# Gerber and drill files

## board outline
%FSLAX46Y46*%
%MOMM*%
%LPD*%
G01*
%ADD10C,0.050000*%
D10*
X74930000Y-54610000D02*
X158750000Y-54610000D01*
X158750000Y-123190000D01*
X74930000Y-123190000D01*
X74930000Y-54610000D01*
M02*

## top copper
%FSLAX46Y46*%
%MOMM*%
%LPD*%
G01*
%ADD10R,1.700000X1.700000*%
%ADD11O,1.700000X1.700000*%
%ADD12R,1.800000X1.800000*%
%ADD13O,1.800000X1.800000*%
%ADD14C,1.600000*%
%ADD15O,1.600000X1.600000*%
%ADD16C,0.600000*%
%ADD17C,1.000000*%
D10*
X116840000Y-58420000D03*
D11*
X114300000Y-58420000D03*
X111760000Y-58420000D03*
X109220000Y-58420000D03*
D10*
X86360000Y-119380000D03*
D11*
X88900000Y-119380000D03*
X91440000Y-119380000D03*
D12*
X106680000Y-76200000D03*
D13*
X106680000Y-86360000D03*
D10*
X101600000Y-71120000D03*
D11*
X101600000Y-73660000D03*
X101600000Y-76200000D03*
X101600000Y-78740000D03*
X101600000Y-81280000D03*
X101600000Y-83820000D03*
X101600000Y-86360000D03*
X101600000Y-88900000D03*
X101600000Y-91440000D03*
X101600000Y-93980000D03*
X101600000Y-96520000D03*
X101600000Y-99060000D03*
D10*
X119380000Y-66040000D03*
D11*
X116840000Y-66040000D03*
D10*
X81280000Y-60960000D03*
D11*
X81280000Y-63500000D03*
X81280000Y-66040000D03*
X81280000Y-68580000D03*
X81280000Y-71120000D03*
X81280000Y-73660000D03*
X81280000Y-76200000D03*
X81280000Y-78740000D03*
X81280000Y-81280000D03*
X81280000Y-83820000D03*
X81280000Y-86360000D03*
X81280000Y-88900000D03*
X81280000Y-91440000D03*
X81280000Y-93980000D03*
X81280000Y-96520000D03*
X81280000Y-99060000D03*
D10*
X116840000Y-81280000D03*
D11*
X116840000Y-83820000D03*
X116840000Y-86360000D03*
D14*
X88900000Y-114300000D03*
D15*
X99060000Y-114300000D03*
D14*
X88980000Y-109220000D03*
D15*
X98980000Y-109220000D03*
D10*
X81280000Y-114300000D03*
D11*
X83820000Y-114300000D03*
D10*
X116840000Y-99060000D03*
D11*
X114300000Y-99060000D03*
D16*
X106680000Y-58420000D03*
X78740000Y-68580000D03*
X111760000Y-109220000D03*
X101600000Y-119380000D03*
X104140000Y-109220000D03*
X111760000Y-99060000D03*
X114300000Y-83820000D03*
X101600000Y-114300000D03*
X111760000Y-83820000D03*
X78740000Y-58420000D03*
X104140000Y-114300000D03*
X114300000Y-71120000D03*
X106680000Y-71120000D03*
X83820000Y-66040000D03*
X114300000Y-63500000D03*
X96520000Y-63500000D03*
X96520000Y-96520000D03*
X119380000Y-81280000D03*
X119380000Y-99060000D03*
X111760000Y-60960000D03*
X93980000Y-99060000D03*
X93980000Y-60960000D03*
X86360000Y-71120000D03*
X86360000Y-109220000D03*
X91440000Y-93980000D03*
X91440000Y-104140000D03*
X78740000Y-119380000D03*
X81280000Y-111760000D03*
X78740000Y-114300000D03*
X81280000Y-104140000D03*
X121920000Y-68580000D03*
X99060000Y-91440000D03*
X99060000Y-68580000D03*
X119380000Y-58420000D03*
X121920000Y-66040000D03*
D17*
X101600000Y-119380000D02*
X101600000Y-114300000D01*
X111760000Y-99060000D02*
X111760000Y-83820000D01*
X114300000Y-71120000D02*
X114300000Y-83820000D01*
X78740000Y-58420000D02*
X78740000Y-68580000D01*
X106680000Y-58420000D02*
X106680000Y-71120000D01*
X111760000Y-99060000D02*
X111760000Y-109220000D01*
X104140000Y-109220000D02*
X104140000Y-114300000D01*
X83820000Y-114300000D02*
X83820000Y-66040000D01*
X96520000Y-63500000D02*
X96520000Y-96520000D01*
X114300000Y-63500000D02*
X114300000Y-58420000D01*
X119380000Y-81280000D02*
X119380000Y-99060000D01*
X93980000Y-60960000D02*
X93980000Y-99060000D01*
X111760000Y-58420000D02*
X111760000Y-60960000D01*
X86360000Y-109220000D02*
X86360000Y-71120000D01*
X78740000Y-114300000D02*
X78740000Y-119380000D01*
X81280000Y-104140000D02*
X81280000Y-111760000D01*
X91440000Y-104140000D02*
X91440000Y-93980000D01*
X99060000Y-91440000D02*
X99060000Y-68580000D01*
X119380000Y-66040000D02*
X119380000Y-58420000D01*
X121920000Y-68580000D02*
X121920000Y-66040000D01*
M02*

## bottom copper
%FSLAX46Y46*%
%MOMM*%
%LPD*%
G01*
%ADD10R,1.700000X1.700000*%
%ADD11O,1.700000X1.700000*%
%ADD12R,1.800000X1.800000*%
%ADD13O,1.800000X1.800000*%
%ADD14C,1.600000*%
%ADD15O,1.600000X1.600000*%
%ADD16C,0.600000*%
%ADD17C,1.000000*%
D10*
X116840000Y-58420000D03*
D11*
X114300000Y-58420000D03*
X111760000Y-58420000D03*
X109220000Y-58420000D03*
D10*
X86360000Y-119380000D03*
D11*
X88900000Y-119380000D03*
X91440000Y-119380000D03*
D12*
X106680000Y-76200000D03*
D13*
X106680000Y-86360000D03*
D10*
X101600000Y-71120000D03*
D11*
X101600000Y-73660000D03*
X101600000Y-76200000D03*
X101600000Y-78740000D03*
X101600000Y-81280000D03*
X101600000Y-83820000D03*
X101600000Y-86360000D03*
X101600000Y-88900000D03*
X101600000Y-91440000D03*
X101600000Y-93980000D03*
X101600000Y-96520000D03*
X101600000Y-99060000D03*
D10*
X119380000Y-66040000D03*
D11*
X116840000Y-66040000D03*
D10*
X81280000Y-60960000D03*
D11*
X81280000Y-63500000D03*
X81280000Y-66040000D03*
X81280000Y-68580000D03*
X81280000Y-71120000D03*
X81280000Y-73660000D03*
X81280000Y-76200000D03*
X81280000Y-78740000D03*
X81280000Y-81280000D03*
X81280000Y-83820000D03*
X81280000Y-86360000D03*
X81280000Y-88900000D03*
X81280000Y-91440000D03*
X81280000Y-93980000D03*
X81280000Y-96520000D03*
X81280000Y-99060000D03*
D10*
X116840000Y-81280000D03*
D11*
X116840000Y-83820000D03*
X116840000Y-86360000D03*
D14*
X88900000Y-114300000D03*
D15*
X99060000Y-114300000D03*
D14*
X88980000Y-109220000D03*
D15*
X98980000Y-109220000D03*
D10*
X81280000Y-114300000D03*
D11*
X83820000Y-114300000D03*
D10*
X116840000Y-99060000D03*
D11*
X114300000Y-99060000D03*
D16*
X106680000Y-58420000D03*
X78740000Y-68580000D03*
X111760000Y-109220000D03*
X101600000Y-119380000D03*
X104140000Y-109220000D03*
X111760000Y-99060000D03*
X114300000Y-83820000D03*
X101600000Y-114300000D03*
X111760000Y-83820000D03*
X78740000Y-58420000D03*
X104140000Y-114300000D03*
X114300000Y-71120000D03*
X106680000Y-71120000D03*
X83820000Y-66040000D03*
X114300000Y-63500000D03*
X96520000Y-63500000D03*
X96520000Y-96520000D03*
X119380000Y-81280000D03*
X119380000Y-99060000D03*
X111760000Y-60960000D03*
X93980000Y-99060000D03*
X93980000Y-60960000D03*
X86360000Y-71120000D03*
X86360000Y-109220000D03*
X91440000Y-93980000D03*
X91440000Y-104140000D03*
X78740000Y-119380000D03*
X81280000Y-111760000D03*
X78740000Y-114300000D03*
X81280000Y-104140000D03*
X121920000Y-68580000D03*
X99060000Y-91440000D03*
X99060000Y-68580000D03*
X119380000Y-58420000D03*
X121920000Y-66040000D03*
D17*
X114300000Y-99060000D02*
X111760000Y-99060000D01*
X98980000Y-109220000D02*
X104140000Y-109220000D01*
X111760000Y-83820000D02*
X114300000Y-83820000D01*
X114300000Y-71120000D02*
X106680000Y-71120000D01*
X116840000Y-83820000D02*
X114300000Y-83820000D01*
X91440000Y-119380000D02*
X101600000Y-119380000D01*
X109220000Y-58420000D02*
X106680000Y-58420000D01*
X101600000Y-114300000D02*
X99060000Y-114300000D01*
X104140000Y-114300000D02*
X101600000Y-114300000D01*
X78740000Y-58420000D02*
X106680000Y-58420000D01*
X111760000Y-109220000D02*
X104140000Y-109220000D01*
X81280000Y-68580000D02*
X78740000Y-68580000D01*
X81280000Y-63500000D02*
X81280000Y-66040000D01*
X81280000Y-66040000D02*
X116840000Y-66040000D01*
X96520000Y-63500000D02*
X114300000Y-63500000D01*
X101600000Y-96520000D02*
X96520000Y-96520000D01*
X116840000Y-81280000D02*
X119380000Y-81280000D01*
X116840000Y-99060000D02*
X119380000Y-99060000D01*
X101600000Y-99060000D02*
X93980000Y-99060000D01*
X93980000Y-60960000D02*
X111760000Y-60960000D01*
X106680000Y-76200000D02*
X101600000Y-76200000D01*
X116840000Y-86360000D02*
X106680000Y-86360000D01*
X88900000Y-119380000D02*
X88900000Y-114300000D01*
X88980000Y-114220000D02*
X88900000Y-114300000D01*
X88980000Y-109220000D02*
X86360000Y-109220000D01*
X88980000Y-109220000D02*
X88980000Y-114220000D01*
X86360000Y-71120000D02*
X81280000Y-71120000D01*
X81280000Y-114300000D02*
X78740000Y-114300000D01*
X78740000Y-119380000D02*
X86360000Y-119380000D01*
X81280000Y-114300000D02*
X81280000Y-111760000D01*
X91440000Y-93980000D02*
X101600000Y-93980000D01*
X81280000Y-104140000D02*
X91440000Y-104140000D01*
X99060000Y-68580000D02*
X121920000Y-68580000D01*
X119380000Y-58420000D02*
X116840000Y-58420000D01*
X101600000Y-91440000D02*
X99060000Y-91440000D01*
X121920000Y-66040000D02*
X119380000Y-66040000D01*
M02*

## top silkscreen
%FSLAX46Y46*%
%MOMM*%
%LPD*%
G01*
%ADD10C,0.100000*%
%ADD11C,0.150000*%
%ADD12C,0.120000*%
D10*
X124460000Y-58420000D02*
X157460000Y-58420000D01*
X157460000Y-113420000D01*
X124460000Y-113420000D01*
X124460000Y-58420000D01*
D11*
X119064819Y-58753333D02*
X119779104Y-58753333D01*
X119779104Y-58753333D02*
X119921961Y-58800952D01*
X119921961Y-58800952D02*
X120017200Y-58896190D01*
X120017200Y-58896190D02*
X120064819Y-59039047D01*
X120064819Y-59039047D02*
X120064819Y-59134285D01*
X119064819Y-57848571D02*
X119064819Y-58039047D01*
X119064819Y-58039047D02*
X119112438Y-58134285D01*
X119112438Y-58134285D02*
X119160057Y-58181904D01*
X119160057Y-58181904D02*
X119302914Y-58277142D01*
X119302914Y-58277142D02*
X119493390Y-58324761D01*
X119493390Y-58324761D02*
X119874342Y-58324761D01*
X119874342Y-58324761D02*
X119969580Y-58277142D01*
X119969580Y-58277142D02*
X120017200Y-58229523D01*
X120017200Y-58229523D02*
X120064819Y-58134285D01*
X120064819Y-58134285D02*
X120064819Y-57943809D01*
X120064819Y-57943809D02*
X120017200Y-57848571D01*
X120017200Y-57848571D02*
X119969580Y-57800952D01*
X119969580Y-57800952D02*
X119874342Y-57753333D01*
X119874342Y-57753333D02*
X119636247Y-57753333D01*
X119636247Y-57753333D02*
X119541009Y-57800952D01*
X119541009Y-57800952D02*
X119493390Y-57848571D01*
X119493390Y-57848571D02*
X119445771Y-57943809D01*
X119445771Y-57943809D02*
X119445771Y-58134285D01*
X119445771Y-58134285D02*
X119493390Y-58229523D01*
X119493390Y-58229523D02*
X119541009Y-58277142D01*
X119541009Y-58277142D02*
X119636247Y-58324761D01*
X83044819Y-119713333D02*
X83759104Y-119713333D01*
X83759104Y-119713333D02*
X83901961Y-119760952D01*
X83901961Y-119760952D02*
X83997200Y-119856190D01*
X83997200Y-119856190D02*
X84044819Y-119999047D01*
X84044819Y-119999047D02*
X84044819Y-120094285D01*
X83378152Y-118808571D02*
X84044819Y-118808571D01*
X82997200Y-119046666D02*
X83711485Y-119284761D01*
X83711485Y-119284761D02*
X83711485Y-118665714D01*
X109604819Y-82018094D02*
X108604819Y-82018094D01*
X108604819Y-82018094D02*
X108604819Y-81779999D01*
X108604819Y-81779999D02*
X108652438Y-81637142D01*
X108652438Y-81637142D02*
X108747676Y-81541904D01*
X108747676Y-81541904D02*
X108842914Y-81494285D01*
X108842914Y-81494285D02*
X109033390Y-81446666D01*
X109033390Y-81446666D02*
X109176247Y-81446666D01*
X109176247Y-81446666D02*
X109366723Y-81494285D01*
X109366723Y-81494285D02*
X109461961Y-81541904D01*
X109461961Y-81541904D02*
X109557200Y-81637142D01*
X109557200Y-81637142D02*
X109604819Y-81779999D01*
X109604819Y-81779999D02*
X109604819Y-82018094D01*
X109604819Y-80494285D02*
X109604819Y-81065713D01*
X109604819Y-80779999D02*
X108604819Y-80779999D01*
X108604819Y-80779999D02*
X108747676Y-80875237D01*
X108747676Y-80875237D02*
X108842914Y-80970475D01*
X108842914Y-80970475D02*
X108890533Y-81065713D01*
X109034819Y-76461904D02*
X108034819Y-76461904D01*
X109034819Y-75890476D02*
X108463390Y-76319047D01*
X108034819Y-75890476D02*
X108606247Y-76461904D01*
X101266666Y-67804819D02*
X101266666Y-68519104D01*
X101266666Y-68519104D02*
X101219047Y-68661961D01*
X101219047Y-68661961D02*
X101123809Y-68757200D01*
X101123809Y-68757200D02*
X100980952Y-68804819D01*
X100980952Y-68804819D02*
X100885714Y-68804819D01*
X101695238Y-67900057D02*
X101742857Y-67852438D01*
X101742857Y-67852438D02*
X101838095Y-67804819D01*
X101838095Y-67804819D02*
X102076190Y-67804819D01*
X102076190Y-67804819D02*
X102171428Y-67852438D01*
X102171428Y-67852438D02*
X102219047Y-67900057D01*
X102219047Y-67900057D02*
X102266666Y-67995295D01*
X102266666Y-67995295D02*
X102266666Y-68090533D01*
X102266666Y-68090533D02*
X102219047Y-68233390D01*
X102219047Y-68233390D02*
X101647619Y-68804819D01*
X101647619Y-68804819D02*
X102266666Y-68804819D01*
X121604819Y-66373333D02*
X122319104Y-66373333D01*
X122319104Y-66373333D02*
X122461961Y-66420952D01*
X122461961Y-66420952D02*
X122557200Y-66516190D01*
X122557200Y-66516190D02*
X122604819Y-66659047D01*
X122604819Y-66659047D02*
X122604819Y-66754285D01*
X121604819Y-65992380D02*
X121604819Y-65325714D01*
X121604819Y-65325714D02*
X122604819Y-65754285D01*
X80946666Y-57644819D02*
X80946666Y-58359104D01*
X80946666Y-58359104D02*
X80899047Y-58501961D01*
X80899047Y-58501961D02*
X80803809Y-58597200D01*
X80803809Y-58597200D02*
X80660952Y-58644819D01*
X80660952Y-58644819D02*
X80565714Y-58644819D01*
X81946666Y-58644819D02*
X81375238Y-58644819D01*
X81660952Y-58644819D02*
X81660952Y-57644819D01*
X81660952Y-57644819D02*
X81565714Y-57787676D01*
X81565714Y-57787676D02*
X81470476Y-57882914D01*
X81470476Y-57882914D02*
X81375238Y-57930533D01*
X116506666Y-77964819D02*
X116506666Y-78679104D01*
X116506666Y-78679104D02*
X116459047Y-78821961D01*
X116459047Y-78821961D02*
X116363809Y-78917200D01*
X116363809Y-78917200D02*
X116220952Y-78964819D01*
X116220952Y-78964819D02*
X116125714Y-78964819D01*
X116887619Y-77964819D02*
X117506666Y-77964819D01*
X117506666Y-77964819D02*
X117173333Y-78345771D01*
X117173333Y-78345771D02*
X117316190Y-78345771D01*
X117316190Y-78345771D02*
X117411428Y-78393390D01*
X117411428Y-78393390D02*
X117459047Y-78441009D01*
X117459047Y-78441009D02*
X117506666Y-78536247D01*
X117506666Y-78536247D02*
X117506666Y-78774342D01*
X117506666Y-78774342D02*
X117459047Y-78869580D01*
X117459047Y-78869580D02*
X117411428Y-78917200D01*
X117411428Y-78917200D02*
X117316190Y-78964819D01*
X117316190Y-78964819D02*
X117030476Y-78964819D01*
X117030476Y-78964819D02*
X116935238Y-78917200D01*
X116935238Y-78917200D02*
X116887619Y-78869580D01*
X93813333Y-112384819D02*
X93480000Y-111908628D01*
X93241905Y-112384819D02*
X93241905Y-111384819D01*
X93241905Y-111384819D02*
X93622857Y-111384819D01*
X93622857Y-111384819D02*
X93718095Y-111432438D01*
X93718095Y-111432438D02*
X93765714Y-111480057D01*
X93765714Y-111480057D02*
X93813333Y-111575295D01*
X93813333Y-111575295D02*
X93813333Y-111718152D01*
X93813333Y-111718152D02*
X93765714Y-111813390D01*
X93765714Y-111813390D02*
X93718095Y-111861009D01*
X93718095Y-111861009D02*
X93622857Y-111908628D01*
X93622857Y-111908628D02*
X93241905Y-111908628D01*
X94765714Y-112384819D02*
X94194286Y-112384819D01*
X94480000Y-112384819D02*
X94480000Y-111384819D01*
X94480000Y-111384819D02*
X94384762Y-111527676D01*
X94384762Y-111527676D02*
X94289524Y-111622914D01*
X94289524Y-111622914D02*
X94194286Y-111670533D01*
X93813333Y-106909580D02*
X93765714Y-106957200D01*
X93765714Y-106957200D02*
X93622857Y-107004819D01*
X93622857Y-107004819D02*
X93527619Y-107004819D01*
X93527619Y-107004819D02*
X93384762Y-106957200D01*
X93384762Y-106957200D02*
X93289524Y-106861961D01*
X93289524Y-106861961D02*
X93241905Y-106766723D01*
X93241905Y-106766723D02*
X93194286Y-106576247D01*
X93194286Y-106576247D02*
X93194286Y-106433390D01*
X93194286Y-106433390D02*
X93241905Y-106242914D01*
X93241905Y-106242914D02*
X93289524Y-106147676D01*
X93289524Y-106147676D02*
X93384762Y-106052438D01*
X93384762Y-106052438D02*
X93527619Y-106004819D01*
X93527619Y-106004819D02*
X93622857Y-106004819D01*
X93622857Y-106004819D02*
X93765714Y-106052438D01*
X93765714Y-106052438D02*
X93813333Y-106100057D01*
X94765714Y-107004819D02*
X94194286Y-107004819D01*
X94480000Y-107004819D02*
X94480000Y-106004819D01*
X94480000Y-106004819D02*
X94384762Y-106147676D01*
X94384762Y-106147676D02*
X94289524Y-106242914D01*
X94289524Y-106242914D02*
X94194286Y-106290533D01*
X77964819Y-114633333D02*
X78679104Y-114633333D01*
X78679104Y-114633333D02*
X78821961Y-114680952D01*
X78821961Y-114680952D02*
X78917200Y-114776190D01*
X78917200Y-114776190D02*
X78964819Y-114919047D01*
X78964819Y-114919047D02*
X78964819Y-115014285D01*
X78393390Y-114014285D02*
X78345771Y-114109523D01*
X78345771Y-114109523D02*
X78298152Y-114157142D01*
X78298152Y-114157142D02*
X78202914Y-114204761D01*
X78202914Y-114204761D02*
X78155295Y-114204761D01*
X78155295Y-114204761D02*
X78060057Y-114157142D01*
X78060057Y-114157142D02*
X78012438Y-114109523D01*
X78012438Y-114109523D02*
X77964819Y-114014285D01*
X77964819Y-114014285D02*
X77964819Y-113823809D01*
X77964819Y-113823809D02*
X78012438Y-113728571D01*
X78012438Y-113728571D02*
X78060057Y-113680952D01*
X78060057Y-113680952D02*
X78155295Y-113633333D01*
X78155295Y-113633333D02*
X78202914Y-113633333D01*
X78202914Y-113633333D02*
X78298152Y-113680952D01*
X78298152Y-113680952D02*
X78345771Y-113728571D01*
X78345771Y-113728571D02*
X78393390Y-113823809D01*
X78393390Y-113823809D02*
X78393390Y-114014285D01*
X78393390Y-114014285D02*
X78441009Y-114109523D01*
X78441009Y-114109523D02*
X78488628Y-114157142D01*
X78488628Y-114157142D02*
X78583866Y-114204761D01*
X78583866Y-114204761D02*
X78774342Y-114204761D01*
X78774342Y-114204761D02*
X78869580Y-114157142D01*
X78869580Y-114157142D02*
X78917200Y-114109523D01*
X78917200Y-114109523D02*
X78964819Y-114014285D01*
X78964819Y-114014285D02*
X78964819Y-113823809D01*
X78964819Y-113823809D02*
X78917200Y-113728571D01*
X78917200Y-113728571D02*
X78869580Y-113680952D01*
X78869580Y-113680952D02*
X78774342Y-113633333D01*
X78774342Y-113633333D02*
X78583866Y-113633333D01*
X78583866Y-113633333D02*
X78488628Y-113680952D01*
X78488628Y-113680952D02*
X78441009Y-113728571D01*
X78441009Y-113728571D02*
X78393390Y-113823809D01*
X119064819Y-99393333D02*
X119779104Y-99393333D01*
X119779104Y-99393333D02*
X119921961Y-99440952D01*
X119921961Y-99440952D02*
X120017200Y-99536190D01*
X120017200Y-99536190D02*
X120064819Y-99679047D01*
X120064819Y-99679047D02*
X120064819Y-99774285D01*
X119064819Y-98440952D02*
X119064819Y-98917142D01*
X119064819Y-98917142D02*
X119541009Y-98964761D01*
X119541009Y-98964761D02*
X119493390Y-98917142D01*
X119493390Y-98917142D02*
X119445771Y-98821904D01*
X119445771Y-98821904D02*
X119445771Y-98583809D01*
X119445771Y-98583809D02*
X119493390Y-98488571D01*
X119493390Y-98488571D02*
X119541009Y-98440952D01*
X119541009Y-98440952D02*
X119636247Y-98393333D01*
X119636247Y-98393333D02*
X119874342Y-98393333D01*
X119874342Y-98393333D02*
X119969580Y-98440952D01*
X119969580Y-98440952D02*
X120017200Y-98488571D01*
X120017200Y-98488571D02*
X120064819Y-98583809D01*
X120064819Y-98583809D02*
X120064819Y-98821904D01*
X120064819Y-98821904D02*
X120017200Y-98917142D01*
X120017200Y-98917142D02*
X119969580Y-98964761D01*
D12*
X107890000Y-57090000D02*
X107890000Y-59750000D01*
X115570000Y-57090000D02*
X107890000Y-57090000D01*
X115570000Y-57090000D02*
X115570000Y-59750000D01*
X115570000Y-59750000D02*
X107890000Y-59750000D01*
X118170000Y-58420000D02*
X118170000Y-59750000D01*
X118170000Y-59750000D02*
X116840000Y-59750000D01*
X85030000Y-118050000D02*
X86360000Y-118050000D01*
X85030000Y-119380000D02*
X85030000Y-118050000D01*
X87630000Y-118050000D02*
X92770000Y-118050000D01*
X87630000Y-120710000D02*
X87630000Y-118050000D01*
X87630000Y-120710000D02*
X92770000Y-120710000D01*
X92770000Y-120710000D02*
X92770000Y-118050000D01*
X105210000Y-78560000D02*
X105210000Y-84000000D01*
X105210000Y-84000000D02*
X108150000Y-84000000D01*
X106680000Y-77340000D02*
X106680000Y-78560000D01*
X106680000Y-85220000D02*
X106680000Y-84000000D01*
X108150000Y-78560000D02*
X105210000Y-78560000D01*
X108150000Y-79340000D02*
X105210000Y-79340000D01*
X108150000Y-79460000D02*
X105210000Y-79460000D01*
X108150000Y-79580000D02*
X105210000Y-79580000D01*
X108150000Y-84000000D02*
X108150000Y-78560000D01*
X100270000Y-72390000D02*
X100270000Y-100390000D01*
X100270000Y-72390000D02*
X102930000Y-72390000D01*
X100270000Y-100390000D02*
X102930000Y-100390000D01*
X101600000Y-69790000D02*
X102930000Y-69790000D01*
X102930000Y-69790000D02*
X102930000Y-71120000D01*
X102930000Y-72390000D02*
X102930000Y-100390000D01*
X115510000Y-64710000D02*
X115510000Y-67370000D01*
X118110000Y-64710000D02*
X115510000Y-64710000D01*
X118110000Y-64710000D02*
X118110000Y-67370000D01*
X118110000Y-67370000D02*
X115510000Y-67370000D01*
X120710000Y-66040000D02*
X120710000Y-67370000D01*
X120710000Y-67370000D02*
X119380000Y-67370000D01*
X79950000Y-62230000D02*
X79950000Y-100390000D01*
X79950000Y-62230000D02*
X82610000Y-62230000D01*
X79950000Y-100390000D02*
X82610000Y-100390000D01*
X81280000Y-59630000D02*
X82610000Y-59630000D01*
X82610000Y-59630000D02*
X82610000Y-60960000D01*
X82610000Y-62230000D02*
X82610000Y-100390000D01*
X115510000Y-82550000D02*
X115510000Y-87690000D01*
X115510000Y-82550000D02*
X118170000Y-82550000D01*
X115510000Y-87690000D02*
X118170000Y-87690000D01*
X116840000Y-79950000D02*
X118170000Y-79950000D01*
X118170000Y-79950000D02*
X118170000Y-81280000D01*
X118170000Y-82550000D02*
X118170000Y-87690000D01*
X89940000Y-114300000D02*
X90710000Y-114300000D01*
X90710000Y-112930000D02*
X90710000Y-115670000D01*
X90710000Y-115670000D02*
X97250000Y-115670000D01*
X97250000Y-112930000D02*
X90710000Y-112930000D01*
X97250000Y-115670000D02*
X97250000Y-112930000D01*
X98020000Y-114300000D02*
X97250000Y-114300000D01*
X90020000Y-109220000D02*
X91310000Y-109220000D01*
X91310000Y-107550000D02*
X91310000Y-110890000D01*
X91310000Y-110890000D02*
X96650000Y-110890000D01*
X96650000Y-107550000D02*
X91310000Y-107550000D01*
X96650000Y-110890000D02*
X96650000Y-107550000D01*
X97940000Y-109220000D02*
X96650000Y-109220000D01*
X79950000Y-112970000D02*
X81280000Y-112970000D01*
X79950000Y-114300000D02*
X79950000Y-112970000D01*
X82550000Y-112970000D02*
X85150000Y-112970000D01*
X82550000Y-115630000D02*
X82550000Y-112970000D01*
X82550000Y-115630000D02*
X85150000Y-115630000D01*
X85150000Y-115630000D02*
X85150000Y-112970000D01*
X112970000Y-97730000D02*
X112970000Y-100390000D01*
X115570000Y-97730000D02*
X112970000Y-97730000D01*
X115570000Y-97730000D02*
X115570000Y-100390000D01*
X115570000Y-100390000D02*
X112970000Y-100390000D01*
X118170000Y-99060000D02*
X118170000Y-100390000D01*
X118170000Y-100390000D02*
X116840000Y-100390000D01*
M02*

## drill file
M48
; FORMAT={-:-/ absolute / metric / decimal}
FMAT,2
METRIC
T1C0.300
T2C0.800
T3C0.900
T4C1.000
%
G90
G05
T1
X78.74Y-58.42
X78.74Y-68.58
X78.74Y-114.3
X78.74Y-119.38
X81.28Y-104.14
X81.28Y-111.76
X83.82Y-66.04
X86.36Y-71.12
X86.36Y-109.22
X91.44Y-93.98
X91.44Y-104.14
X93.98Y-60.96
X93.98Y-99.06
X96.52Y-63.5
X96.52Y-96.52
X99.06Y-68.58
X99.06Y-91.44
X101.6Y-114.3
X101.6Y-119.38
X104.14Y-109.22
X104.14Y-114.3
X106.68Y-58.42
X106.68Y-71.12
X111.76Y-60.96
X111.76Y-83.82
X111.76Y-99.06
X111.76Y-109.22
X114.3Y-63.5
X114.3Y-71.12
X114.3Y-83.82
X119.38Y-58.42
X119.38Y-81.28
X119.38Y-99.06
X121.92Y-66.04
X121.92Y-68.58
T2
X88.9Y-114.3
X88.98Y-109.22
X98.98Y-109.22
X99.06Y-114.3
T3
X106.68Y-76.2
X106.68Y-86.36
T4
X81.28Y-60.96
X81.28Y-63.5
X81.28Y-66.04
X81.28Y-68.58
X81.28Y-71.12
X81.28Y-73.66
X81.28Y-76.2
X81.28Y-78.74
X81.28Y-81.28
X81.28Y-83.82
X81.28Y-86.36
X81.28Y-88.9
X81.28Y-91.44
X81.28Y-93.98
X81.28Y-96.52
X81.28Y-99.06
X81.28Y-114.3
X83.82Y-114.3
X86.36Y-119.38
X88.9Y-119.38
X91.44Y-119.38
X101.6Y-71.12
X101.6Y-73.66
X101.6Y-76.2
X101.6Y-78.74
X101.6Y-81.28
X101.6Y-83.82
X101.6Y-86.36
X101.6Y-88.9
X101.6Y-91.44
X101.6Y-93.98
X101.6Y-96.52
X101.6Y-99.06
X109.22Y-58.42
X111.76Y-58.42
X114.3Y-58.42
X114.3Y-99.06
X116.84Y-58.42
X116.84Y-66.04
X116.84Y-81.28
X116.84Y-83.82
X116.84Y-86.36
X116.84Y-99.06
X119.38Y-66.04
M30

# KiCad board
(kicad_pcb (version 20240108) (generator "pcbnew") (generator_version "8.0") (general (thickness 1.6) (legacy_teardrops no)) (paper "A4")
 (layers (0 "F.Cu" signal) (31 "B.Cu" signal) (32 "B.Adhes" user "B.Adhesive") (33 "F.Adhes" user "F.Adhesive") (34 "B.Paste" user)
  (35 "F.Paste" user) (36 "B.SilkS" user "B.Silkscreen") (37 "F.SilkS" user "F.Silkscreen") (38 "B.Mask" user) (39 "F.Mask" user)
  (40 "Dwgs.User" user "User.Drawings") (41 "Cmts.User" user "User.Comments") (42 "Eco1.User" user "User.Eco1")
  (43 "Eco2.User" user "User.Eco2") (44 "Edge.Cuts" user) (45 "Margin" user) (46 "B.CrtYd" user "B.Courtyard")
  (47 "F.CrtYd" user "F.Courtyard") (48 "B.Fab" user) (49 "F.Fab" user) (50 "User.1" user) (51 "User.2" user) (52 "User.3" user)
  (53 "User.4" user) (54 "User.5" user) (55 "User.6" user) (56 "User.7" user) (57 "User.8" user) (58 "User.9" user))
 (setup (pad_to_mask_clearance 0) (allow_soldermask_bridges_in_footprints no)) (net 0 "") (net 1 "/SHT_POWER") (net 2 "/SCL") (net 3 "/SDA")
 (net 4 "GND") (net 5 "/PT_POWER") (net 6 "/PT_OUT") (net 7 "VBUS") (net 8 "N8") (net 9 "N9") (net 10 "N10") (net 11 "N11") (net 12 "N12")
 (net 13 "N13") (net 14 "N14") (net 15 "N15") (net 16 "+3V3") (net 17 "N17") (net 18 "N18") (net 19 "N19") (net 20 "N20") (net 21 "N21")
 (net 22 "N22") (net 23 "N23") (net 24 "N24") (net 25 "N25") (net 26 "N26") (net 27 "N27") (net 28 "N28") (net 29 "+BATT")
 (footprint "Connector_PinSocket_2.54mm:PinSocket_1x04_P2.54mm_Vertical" (layer "F.Cu") (at 116.84 58.42 -90)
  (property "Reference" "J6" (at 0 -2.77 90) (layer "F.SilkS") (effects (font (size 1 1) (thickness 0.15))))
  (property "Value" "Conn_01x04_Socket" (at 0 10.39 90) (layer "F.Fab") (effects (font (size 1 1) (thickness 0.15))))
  (fp_line (start -1.33 8.95) (end 1.33 8.95) (stroke (width 0.12) (type solid)) (layer "F.SilkS"))
  (fp_line (start -1.33 1.27) (end -1.33 8.95) (stroke (width 0.12) (type solid)) (layer "F.SilkS"))
  (fp_line (start -1.33 1.27) (end 1.33 1.27) (stroke (width 0.12) (type solid)) (layer "F.SilkS"))
  (fp_line (start 1.33 1.27) (end 1.33 8.95) (stroke (width 0.12) (type solid)) (layer "F.SilkS"))
  (fp_line (start 0 -1.33) (end 1.33 -1.33) (stroke (width 0.12) (type solid)) (layer "F.SilkS"))
  (fp_line (start 1.33 -1.33) (end 1.33 0) (stroke (width 0.12) (type solid)) (layer "F.SilkS"))
  (pad "1" thru_hole rect (at 0 0 270) (size 1.7 1.7) (drill 1) (layers "*.Cu" "*.Mask") (remove_unused_layers no) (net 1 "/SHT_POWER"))
  (pad "2" thru_hole oval (at 0 2.54 270) (size 1.7 1.7) (drill 1) (layers "*.Cu" "*.Mask") (remove_unused_layers no) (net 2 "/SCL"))
  (pad "3" thru_hole oval (at 0 5.08 270) (size 1.7 1.7) (drill 1) (layers "*.Cu" "*.Mask") (remove_unused_layers no) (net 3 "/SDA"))
  (pad "4" thru_hole oval (at 0 7.62 270) (size 1.7 1.7) (drill 1) (layers "*.Cu" "*.Mask") (remove_unused_layers no) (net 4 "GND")))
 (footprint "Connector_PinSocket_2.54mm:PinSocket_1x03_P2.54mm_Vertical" (layer "F.Cu") (at 86.36 119.38 90)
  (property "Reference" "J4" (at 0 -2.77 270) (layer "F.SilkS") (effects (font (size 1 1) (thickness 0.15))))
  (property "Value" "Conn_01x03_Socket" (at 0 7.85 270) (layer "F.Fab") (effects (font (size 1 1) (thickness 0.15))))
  (fp_line (start 1.33 -1.33) (end 1.33 0) (stroke (width 0.12) (type solid)) (layer "F.SilkS"))
  (fp_line (start 0 -1.33) (end 1.33 -1.33) (stroke (width 0.12) (type solid)) (layer "F.SilkS"))
  (fp_line (start 1.33 1.27) (end 1.33 6.41) (stroke (width 0.12) (type solid)) (layer "F.SilkS"))
  (fp_line (start -1.33 1.27) (end 1.33 1.27) (stroke (width 0.12) (type solid)) (layer "F.SilkS"))
  (fp_line (start -1.33 1.27) (end -1.33 6.41) (stroke (width 0.12) (type solid)) (layer "F.SilkS"))
  (fp_line (start -1.33 6.41) (end 1.33 6.41) (stroke (width 0.12) (type solid)) (layer "F.SilkS"))
  (pad "1" thru_hole rect (at 0 0 90) (size 1.7 1.7) (drill 1) (layers "*.Cu" "*.Mask") (remove_unused_layers no) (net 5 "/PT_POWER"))
  (pad "2" thru_hole oval (at 0 2.54 90) (size 1.7 1.7) (drill 1) (layers "*.Cu" "*.Mask") (remove_unused_layers no) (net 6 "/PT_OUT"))
  (pad "3" thru_hole oval (at 0 5.08 90) (size 1.7 1.7) (drill 1) (layers "*.Cu" "*.Mask") (remove_unused_layers no) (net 4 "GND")))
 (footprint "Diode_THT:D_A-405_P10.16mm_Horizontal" (layer "F.Cu") (at 106.68 76.2 -90)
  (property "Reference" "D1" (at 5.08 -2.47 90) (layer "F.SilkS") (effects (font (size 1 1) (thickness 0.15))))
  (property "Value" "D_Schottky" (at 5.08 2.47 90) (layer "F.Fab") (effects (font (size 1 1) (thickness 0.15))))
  (fp_line (start 2.36 1.47) (end 7.8 1.47) (stroke (width 0.12) (type solid)) (layer "F.SilkS"))
  (fp_line (start 7.8 1.47) (end 7.8 -1.47) (stroke (width 0.12) (type solid)) (layer "F.SilkS"))
  (fp_line (start 1.14 0) (end 2.36 0) (stroke (width 0.12) (type solid)) (layer "F.SilkS"))
  (fp_line (start 9.02 0) (end 7.8 0) (stroke (width 0.12) (type solid)) (layer "F.SilkS"))
  (fp_line (start 2.36 -1.47) (end 2.36 1.47) (stroke (width 0.12) (type solid)) (layer "F.SilkS"))
  (fp_line (start 3.14 -1.47) (end 3.14 1.47) (stroke (width 0.12) (type solid)) (layer "F.SilkS"))
  (fp_line (start 3.26 -1.47) (end 3.26 1.47) (stroke (width 0.12) (type solid)) (layer "F.SilkS"))
  (fp_line (start 3.38 -1.47) (end 3.38 1.47) (stroke (width 0.12) (type solid)) (layer "F.SilkS"))
  (fp_line (start 7.8 -1.47) (end 2.36 -1.47) (stroke (width 0.12) (type solid)) (layer "F.SilkS"))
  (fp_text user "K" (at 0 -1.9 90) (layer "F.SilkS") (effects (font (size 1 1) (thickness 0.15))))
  (pad "1" thru_hole rect (at 0 0 270) (size 1.8 1.8) (drill 0.9) (layers "*.Cu" "*.Mask") (remove_unused_layers no) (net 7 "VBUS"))
  (pad "2" thru_hole oval (at 10.16 0 270) (size 1.8 1.8) (drill 0.9) (layers "*.Cu" "*.Mask") (remove_unused_layers no) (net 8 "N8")))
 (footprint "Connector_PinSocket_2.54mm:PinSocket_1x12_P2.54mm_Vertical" (layer "F.Cu") (at 101.6 71.12)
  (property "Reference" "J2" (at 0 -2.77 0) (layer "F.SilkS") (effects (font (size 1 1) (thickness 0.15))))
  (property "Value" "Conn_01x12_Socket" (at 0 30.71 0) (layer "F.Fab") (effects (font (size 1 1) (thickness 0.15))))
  (fp_line (start -1.33 1.27) (end -1.33 29.27) (stroke (width 0.12) (type solid)) (layer "F.SilkS"))
  (fp_line (start -1.33 1.27) (end 1.33 1.27) (stroke (width 0.12) (type solid)) (layer "F.SilkS"))
  (fp_line (start -1.33 29.27) (end 1.33 29.27) (stroke (width 0.12) (type solid)) (layer "F.SilkS"))
  (fp_line (start 0 -1.33) (end 1.33 -1.33) (stroke (width 0.12) (type solid)) (layer "F.SilkS"))
  (fp_line (start 1.33 -1.33) (end 1.33 0) (stroke (width 0.12) (type solid)) (layer "F.SilkS"))
  (fp_line (start 1.33 1.27) (end 1.33 29.27) (stroke (width 0.12) (type solid)) (layer "F.SilkS"))
  (pad "1" thru_hole rect (at 0 0) (size 1.7 1.7) (drill 1) (layers "*.Cu" "*.Mask") (remove_unused_layers no) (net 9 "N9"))
  (pad "2" thru_hole oval (at 0 2.54) (size 1.7 1.7) (drill 1) (layers "*.Cu" "*.Mask") (remove_unused_layers no) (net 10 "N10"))
  (pad "3" thru_hole oval (at 0 5.08) (size 1.7 1.7) (drill 1) (layers "*.Cu" "*.Mask") (remove_unused_layers no) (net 7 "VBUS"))
  (pad "4" thru_hole oval (at 0 7.62) (size 1.7 1.7) (drill 1) (layers "*.Cu" "*.Mask") (remove_unused_layers no) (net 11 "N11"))
  (pad "5" thru_hole oval (at 0 10.16) (size 1.7 1.7) (drill 1) (layers "*.Cu" "*.Mask") (remove_unused_layers no) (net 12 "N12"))
  (pad "6" thru_hole oval (at 0 12.7) (size 1.7 1.7) (drill 1) (layers "*.Cu" "*.Mask") (remove_unused_layers no) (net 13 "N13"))
  (pad "7" thru_hole oval (at 0 15.24) (size 1.7 1.7) (drill 1) (layers "*.Cu" "*.Mask") (remove_unused_layers no) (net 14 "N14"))
  (pad "8" thru_hole oval (at 0 17.78) (size 1.7 1.7) (drill 1) (layers "*.Cu" "*.Mask") (remove_unused_layers no) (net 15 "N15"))
  (pad "9" thru_hole oval (at 0 20.32) (size 1.7 1.7) (drill 1) (layers "*.Cu" "*.Mask") (remove_unused_layers no) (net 1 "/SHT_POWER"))
  (pad "10" thru_hole oval (at 0 22.86) (size 1.7 1.7) (drill 1) (layers "*.Cu" "*.Mask") (remove_unused_layers no) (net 5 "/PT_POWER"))
  (pad "11" thru_hole oval (at 0 25.4) (size 1.7 1.7) (drill 1) (layers "*.Cu" "*.Mask") (remove_unused_layers no) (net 2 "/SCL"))
  (pad "12" thru_hole oval (at 0 27.94) (size 1.7 1.7) (drill 1) (layers "*.Cu" "*.Mask") (remove_unused_layers no) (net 3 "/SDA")))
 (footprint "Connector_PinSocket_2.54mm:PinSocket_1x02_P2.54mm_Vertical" (layer "F.Cu") (at 119.38 66.04 -90)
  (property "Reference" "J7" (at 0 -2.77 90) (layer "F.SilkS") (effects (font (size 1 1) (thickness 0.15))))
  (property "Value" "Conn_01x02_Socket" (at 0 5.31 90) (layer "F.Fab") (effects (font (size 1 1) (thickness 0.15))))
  (fp_line (start -1.33 3.87) (end 1.33 3.87) (stroke (width 0.12) (type solid)) (layer "F.SilkS"))
  (fp_line (start -1.33 1.27) (end -1.33 3.87) (stroke (width 0.12) (type solid)) (layer "F.SilkS"))
  (fp_line (start -1.33 1.27) (end 1.33 1.27) (stroke (width 0.12) (type solid)) (layer "F.SilkS"))
  (fp_line (start 1.33 1.27) (end 1.33 3.87) (stroke (width 0.12) (type solid)) (layer "F.SilkS"))
  (fp_line (start 0 -1.33) (end 1.33 -1.33) (stroke (width 0.12) (type solid)) (layer "F.SilkS"))
  (fp_line (start 1.33 -1.33) (end 1.33 0) (stroke (width 0.12) (type solid)) (layer "F.SilkS"))
  (pad "1" thru_hole rect (at 0 0 270) (size 1.7 1.7) (drill 1) (layers "*.Cu" "*.Mask") (remove_unused_layers no) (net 1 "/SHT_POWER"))
  (pad "2" thru_hole oval (at 0 2.54 270) (size 1.7 1.7) (drill 1) (layers "*.Cu" "*.Mask") (remove_unused_layers no) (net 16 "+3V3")))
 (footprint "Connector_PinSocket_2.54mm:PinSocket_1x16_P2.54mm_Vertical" (layer "F.Cu") (at 81.28 60.96)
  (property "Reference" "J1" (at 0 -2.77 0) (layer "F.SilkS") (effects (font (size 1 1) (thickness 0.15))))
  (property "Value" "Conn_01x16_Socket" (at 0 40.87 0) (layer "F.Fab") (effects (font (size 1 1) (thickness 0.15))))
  (fp_line (start -1.33 1.27) (end -1.33 39.43) (stroke (width 0.12) (type solid)) (layer "F.SilkS"))
  (fp_line (start -1.33 1.27) (end 1.33 1.27) (stroke (width 0.12) (type solid)) (layer "F.SilkS"))
  (fp_line (start -1.33 39.43) (end 1.33 39.43) (stroke (width 0.12) (type solid)) (layer "F.SilkS"))
  (fp_line (start 0 -1.33) (end 1.33 -1.33) (stroke (width 0.12) (type solid)) (layer "F.SilkS"))
  (fp_line (start 1.33 -1.33) (end 1.33 0) (stroke (width 0.12) (type solid)) (layer "F.SilkS"))
  (fp_line (start 1.33 1.27) (end 1.33 39.43) (stroke (width 0.12) (type solid)) (layer "F.SilkS"))
  (pad "1" thru_hole rect (at 0 0) (size 1.7 1.7) (drill 1) (layers "*.Cu" "*.Mask") (remove_unused_layers no) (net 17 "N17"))
  (pad "2" thru_hole oval (at 0 2.54) (size 1.7 1.7) (drill 1) (layers "*.Cu" "*.Mask") (remove_unused_layers no) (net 16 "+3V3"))
  (pad "3" thru_hole oval (at 0 5.08) (size 1.7 1.7) (drill 1) (layers "*.Cu" "*.Mask") (remove_unused_layers no) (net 16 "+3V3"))
  (pad "4" thru_hole oval (at 0 7.62) (size 1.7 1.7) (drill 1) (layers "*.Cu" "*.Mask") (remove_unused_layers no) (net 4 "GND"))
  (pad "5" thru_hole oval (at 0 10.16) (size 1.7 1.7) (drill 1) (layers "*.Cu" "*.Mask") (remove_unused_layers no) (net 6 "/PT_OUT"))
  (pad "6" thru_hole oval (at 0 12.7) (size 1.7 1.7) (drill 1) (layers "*.Cu" "*.Mask") (remove_unused_layers no) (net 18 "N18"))
  (pad "7" thru_hole oval (at 0 15.24) (size 1.7 1.7) (drill 1) (layers "*.Cu" "*.Mask") (remove_unused_layers no) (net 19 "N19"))
  (pad "8" thru_hole oval (at 0 17.78) (size 1.7 1.7) (drill 1) (layers "*.Cu" "*.Mask") (remove_unused_layers no) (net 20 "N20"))
  (pad "9" thru_hole oval (at 0 20.32) (size 1.7 1.7) (drill 1) (layers "*.Cu" "*.Mask") (remove_unused_layers no) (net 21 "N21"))
  (pad "10" thru_hole oval (at 0 22.86) (size 1.7 1.7) (drill 1) (layers "*.Cu" "*.Mask") (remove_unused_layers no) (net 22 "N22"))
  (pad "11" thru_hole oval (at 0 25.4) (size 1.7 1.7) (drill 1) (layers "*.Cu" "*.Mask") (remove_unused_layers no) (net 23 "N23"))
  (pad "12" thru_hole oval (at 0 27.94) (size 1.7 1.7) (drill 1) (layers "*.Cu" "*.Mask") (remove_unused_layers no) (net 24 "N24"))
  (pad "13" thru_hole oval (at 0 30.48) (size 1.7 1.7) (drill 1) (layers "*.Cu" "*.Mask") (remove_unused_layers no) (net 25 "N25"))
  (pad "14" thru_hole oval (at 0 33.02) (size 1.7 1.7) (drill 1) (layers "*.Cu" "*.Mask") (remove_unused_layers no) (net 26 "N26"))
  (pad "15" thru_hole oval (at 0 35.56) (size 1.7 1.7) (drill 1) (layers "*.Cu" "*.Mask") (remove_unused_layers no) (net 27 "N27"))
  (pad "16" thru_hole oval (at 0 38.1) (size 1.7 1.7) (drill 1) (layers "*.Cu" "*.Mask") (remove_unused_layers no) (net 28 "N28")))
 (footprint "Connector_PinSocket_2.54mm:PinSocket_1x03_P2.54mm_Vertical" (layer "F.Cu") (at 116.84 81.28)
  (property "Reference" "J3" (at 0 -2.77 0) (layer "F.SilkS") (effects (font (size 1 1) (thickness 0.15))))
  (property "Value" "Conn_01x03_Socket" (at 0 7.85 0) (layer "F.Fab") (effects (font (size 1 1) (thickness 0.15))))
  (fp_line (start -1.33 1.27) (end -1.33 6.41) (stroke (width 0.12) (type solid)) (layer "F.SilkS"))
  (fp_line (start -1.33 1.27) (end 1.33 1.27) (stroke (width 0.12) (type solid)) (layer "F.SilkS"))
  (fp_line (start -1.33 6.41) (end 1.33 6.41) (stroke (width 0.12) (type solid)) (layer "F.SilkS"))
  (fp_line (start 0 -1.33) (end 1.33 -1.33) (stroke (width 0.12) (type solid)) (layer "F.SilkS"))
  (fp_line (start 1.33 -1.33) (end 1.33 0) (stroke (width 0.12) (type solid)) (layer "F.SilkS"))
  (fp_line (start 1.33 1.27) (end 1.33 6.41) (stroke (width 0.12) (type solid)) (layer "F.SilkS"))
  (pad "1" thru_hole rect (at 0 0) (size 1.7 1.7) (drill 1) (layers "*.Cu" "*.Mask") (remove_unused_layers no) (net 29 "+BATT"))
  (pad "2" thru_hole oval (at 0 2.54) (size 1.7 1.7) (drill 1) (layers "*.Cu" "*.Mask") (remove_unused_layers no) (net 4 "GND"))
  (pad "3" thru_hole oval (at 0 5.08) (size 1.7 1.7) (drill 1) (layers "*.Cu" "*.Mask") (remove_unused_layers no) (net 8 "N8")))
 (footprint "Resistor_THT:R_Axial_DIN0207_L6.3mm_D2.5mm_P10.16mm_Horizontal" (layer "F.Cu") (at 88.9 114.3)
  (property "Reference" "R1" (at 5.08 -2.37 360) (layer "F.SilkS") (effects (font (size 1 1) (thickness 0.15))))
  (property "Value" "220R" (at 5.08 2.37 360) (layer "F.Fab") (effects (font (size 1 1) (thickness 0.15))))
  (fp_line (start 1.04 0) (end 1.81 0) (stroke (width 0.12) (type solid)) (layer "F.SilkS"))
  (fp_line (start 1.81 -1.37) (end 1.81 1.37) (stroke (width 0.12) (type solid)) (layer "F.SilkS"))
  (fp_line (start 1.81 1.37) (end 8.35 1.37) (stroke (width 0.12) (type solid)) (layer "F.SilkS"))
  (fp_line (start 8.35 -1.37) (end 1.81 -1.37) (stroke (width 0.12) (type solid)) (layer "F.SilkS"))
  (fp_line (start 8.35 1.37) (end 8.35 -1.37) (stroke (width 0.12) (type solid)) (layer "F.SilkS"))
  (fp_line (start 9.12 0) (end 8.35 0) (stroke (width 0.12) (type solid)) (layer "F.SilkS"))
  (pad "1" thru_hole circle (at 0 0) (size 1.6 1.6) (drill 0.8) (layers "*.Cu" "*.Mask") (remove_unused_layers no) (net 6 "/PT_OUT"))
  (pad "2" thru_hole oval (at 10.16 0) (size 1.6 1.6) (drill 0.8) (layers "*.Cu" "*.Mask") (remove_unused_layers no) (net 4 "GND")))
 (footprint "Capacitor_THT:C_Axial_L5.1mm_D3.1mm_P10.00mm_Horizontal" (layer "F.Cu") (at 88.98 109.22)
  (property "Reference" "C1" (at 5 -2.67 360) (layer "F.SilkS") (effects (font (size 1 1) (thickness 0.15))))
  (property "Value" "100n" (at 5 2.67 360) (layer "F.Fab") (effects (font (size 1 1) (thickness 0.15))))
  (fp_line (start 1.04 0) (end 2.33 0) (stroke (width 0.12) (type solid)) (layer "F.SilkS"))
  (fp_line (start 2.33 -1.67) (end 2.33 1.67) (stroke (width 0.12) (type solid)) (layer "F.SilkS"))
  (fp_line (start 2.33 1.67) (end 7.67 1.67) (stroke (width 0.12) (type solid)) (layer "F.SilkS"))
  (fp_line (start 7.67 -1.67) (end 2.33 -1.67) (stroke (width 0.12) (type solid)) (layer "F.SilkS"))
  (fp_line (start 7.67 1.67) (end 7.67 -1.67) (stroke (width 0.12) (type solid)) (layer "F.SilkS"))
  (fp_line (start 8.96 0) (end 7.67 0) (stroke (width 0.12) (type solid)) (layer "F.SilkS"))
  (pad "1" thru_hole circle (at 0 0) (size 1.6 1.6) (drill 0.8) (layers "*.Cu" "*.Mask") (remove_unused_layers no) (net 6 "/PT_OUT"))
  (pad "2" thru_hole oval (at 10 0) (size 1.6 1.6) (drill 0.8) (layers "*.Cu" "*.Mask") (remove_unused_layers no) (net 4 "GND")))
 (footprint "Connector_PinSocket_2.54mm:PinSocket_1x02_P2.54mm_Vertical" (layer "F.Cu") (at 81.28 114.3 90)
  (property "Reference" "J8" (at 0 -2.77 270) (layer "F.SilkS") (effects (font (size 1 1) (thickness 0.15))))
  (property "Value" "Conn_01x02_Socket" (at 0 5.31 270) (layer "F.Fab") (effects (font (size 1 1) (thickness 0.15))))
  (fp_line (start 1.33 -1.33) (end 1.33 0) (stroke (width 0.12) (type solid)) (layer "F.SilkS"))
  (fp_line (start 0 -1.33) (end 1.33 -1.33) (stroke (width 0.12) (type solid)) (layer "F.SilkS"))
  (fp_line (start 1.33 1.27) (end 1.33 3.87) (stroke (width 0.12) (type solid)) (layer "F.SilkS"))
  (fp_line (start -1.33 1.27) (end 1.33 1.27) (stroke (width 0.12) (type solid)) (layer "F.SilkS"))
  (fp_line (start -1.33 1.27) (end -1.33 3.87) (stroke (width 0.12) (type solid)) (layer "F.SilkS"))
  (fp_line (start -1.33 3.87) (end 1.33 3.87) (stroke (width 0.12) (type solid)) (layer "F.SilkS"))
  (pad "1" thru_hole rect (at 0 0 90) (size 1.7 1.7) (drill 1) (layers "*.Cu" "*.Mask") (remove_unused_layers no) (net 5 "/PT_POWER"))
  (pad "2" thru_hole oval (at 0 2.54 90) (size 1.7 1.7) (drill 1) (layers "*.Cu" "*.Mask") (remove_unused_layers no) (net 16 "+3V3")))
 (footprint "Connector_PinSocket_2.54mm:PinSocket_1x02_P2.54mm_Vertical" (layer "F.Cu") (at 116.84 99.06 -90)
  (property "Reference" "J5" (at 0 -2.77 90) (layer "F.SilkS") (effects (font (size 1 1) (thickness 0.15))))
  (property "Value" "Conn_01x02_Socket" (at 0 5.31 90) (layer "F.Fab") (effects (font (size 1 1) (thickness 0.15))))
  (fp_line (start -1.33 3.87) (end 1.33 3.87) (stroke (width 0.12) (type solid)) (layer "F.SilkS"))
  (fp_line (start -1.33 1.27) (end -1.33 3.87) (stroke (width 0.12) (type solid)) (layer "F.SilkS"))
  (fp_line (start -1.33 1.27) (end 1.33 1.27) (stroke (width 0.12) (type solid)) (layer "F.SilkS"))
  (fp_line (start 1.33 1.27) (end 1.33 3.87) (stroke (width 0.12) (type solid)) (layer "F.SilkS"))
  (fp_line (start 0 -1.33) (end 1.33 -1.33) (stroke (width 0.12) (type solid)) (layer "F.SilkS"))
  (fp_line (start 1.33 -1.33) (end 1.33 0) (stroke (width 0.12) (type solid)) (layer "F.SilkS"))
  (pad "1" thru_hole rect (at 0 0 270) (size 1.7 1.7) (drill 1) (layers "*.Cu" "*.Mask") (remove_unused_layers no) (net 29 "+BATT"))
  (pad "2" thru_hole oval (at 0 2.54 270) (size 1.7 1.7) (drill 1) (layers "*.Cu" "*.Mask") (remove_unused_layers no) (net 4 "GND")))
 (gr_rect (start 124.46 58.42) (end 157.46 113.42) (stroke (width 0.1) (type default)) (fill none) (layer "F.SilkS"))
 (gr_rect (start 74.93 54.61) (end 158.75 123.19) (stroke (width 0.05) (type default)) (fill none) (layer "Edge.Cuts"))
 (segment (start 101.6 119.38) (end 101.6 114.3) (width 1) (layer "F.Cu") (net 4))
 (segment (start 111.76 99.06) (end 111.76 83.82) (width 1) (layer "F.Cu") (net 4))
 (segment (start 114.3 71.12) (end 114.3 83.82) (width 1) (layer "F.Cu") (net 4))
 (segment (start 78.74 58.42) (end 78.74 68.58) (width 1) (layer "F.Cu") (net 4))
 (segment (start 106.68 58.42) (end 106.68 71.12) (width 1) (layer "F.Cu") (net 4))
 (segment (start 111.76 99.06) (end 111.76 109.22) (width 1) (layer "F.Cu") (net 4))
 (segment (start 104.14 109.22) (end 104.14 114.3) (width 1) (layer "F.Cu") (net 4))
 (via (at 106.68 58.42) (size 0.6) (drill 0.3) (layers "F.Cu" "B.Cu") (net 4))
 (via (at 78.74 68.58) (size 0.6) (drill 0.3) (layers "F.Cu" "B.Cu") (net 4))
 (via (at 111.76 109.22) (size 0.6) (drill 0.3) (layers "F.Cu" "B.Cu") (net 4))
 (via (at 101.6 119.38) (size 0.6) (drill 0.3) (layers "F.Cu" "B.Cu") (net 4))
 (via (at 104.14 109.22) (size 0.6) (drill 0.3) (layers "F.Cu" "B.Cu") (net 4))
 (via (at 111.76 99.06) (size 0.6) (drill 0.3) (layers "F.Cu" "B.Cu") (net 4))
 (via (at 114.3 83.82) (size 0.6) (drill 0.3) (layers "F.Cu" "B.Cu") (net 4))
 (via (at 101.6 114.3) (size 0.6) (drill 0.3) (layers "F.Cu" "B.Cu") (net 4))
 (via (at 111.76 83.82) (size 0.6) (drill 0.3) (layers "F.Cu" "B.Cu") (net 4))
 (via (at 78.74 58.42) (size 0.6) (drill 0.3) (layers "F.Cu" "B.Cu") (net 4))
 (via (at 104.14 114.3) (size 0.6) (drill 0.3) (layers "F.Cu" "B.Cu") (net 4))
 (via (at 114.3 71.12) (size 0.6) (drill 0.3) (layers "F.Cu" "B.Cu") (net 4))
 (via (at 106.68 71.12) (size 0.6) (drill 0.3) (layers "F.Cu" "B.Cu") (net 4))
 (segment (start 114.3 99.06) (end 111.76 99.06) (width 1) (layer "B.Cu") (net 4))
 (segment (start 98.98 109.22) (end 104.14 109.22) (width 1) (layer "B.Cu") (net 4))
 (segment (start 111.76 83.82) (end 114.3 83.82) (width 1) (layer "B.Cu") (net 4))
 (segment (start 114.3 71.12) (end 106.68 71.12) (width 1) (layer "B.Cu") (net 4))
 (segment (start 116.84 83.82) (end 114.3 83.82) (width 1) (layer "B.Cu") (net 4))
 (segment (start 91.44 119.38) (end 101.6 119.38) (width 1) (layer "B.Cu") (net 4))
 (segment (start 109.22 58.42) (end 106.68 58.42) (width 1) (layer "B.Cu") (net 4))
 (segment (start 101.6 114.3) (end 99.06 114.3) (width 1) (layer "B.Cu") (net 4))
 (segment (start 104.14 114.3) (end 101.6 114.3) (width 1) (layer "B.Cu") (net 4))
 (segment (start 78.74 58.42) (end 106.68 58.42) (width 1) (layer "B.Cu") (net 4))
 (segment (start 111.76 109.22) (end 104.14 109.22) (width 1) (layer "B.Cu") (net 4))
 (segment (start 81.28 68.58) (end 78.74 68.58) (width 1) (layer "B.Cu") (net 4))
 (segment (start 83.82 114.3) (end 83.82 66.04) (width 1) (layer "F.Cu") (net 16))
 (via (at 83.82 66.04) (size 0.6) (drill 0.3) (layers "F.Cu" "B.Cu") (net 16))
 (segment (start 81.28 63.5) (end 81.28 66.04) (width 1) (layer "B.Cu") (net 16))
 (segment (start 81.28 66.04) (end 116.84 66.04) (width 1) (layer "B.Cu") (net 16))
 (segment (start 96.52 63.5) (end 96.52 96.52) (width 1) (layer "F.Cu") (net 2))
 (segment (start 114.3 63.5) (end 114.3 58.42) (width 1) (layer "F.Cu") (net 2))
 (via (at 114.3 63.5) (size 0.6) (drill 0.3) (layers "F.Cu" "B.Cu") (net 2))
 (via (at 96.52 63.5) (size 0.6) (drill 0.3) (layers "F.Cu" "B.Cu") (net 2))
 (via (at 96.52 96.52) (size 0.6) (drill 0.3) (layers "F.Cu" "B.Cu") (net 2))
 (segment (start 96.52 63.5) (end 114.3 63.5) (width 1) (layer "B.Cu") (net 2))
 (segment (start 101.6 96.52) (end 96.52 96.52) (width 1) (layer "B.Cu") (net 2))
 (segment (start 119.38 81.28) (end 119.38 99.06) (width 1) (layer "F.Cu") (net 29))
 (via (at 119.38 81.28) (size 0.6) (drill 0.3) (layers "F.Cu" "B.Cu") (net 29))
 (via (at 119.38 99.06) (size 0.6) (drill 0.3) (layers "F.Cu" "B.Cu") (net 29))
 (segment (start 116.84 81.28) (end 119.38 81.28) (width 1) (layer "B.Cu") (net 29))
 (segment (start 116.84 99.06) (end 119.38 99.06) (width 1) (layer "B.Cu") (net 29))
 (segment (start 93.98 60.96) (end 93.98 99.06) (width 1) (layer "F.Cu") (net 3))
 (segment (start 111.76 58.42) (end 111.76 60.96) (width 1) (layer "F.Cu") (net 3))
 (via (at 111.76 60.96) (size 0.6) (drill 0.3) (layers "F.Cu" "B.Cu") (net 3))
 (via (at 93.98 99.06) (size 0.6) (drill 0.3) (layers "F.Cu" "B.Cu") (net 3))
 (via (at 93.98 60.96) (size 0.6) (drill 0.3) (layers "F.Cu" "B.Cu") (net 3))
 (segment (start 101.6 99.06) (end 93.98 99.06) (width 1) (layer "B.Cu") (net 3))
 (segment (start 93.98 60.96) (end 111.76 60.96) (width 1) (layer "B.Cu") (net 3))
 (segment (start 106.68 76.2) (end 101.6 76.2) (width 1) (layer "B.Cu") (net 7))
 (segment (start 116.84 86.36) (end 106.68 86.36) (width 1) (layer "B.Cu") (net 8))
 (segment (start 86.36 109.22) (end 86.36 71.12) (width 1) (layer "F.Cu") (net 6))
 (via (at 86.36 71.12) (size 0.6) (drill 0.3) (layers "F.Cu" "B.Cu") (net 6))
 (via (at 86.36 109.22) (size 0.6) (drill 0.3) (layers "F.Cu" "B.Cu") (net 6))
 (segment (start 88.9 119.38) (end 88.9 114.3) (width 1) (layer "B.Cu") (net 6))
 (segment (start 88.98 114.22) (end 88.9 114.3) (width 1) (layer "B.Cu") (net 6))
 (segment (start 88.98 109.22) (end 86.36 109.22) (width 1) (layer "B.Cu") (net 6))
 (segment (start 88.98 109.22) (end 88.98 114.22) (width 1) (layer "B.Cu") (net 6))
 (segment (start 86.36 71.12) (end 81.28 71.12) (width 1) (layer "B.Cu") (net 6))
 (segment (start 78.74 114.3) (end 78.74 119.38) (width 1) (layer "F.Cu") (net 5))
 (segment (start 81.28 104.14) (end 81.28 111.76) (width 1) (layer "F.Cu") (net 5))
 (segment (start 91.44 104.14) (end 91.44 93.98) (width 1) (layer "F.Cu") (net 5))
 (via (at 91.44 93.98) (size 0.6) (drill 0.3) (layers "F.Cu" "B.Cu") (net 5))
 (via (at 91.44 104.14) (size 0.6) (drill 0.3) (layers "F.Cu" "B.Cu") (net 5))
 (via (at 78.74 119.38) (size 0.6) (drill 0.3) (layers "F.Cu" "B.Cu") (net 5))
 (via (at 81.28 111.76) (size 0.6) (drill 0.3) (layers "F.Cu" "B.Cu") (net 5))
 (via (at 78.74 114.3) (size 0.6) (drill 0.3) (layers "F.Cu" "B.Cu") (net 5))
 (via (at 81.28 104.14) (size 0.6) (drill 0.3) (layers "F.Cu" "B.Cu") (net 5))
 (segment (start 81.28 114.3) (end 78.74 114.3) (width 1) (layer "B.Cu") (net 5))
 (segment (start 78.74 119.38) (end 86.36 119.38) (width 1) (layer "B.Cu") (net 5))
 (segment (start 81.28 114.3) (end 81.28 111.76) (width 1) (layer "B.Cu") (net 5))
 (segment (start 91.44 93.98) (end 101.6 93.98) (width 1) (layer "B.Cu") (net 5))
 (segment (start 81.28 104.14) (end 91.44 104.14) (width 1) (layer "B.Cu") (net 5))
 (segment (start 99.06 91.44) (end 99.06 68.58) (width 1) (layer "F.Cu") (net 1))
 (segment (start 119.38 66.04) (end 119.38 58.42) (width 1) (layer "F.Cu") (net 1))
 (segment (start 121.92 68.58) (end 121.92 66.04) (width 1) (layer "F.Cu") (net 1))
 (via (at 121.92 68.58) (size 0.6) (drill 0.3) (layers "F.Cu" "B.Cu") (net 1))
 (via (at 99.06 91.44) (size 0.6) (drill 0.3) (layers "F.Cu" "B.Cu") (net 1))
 (via (at 99.06 68.58) (size 0.6) (drill 0.3) (layers "F.Cu" "B.Cu") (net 1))
 (via (at 119.38 58.42) (size 0.6) (drill 0.3) (layers "F.Cu" "B.Cu") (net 1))
 (via (at 121.92 66.04) (size 0.6) (drill 0.3) (layers "F.Cu" "B.Cu") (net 1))
 (segment (start 99.06 68.58) (end 121.92 68.58) (width 1) (layer "B.Cu") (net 1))
 (segment (start 119.38 58.42) (end 116.84 58.42) (width 1) (layer "B.Cu") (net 1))
 (segment (start 101.6 91.44) (end 99.06 91.44) (width 1) (layer "B.Cu") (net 1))
 (segment (start 121.92 66.04) (end 119.38 66.04) (width 1) (layer "B.Cu") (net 1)))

